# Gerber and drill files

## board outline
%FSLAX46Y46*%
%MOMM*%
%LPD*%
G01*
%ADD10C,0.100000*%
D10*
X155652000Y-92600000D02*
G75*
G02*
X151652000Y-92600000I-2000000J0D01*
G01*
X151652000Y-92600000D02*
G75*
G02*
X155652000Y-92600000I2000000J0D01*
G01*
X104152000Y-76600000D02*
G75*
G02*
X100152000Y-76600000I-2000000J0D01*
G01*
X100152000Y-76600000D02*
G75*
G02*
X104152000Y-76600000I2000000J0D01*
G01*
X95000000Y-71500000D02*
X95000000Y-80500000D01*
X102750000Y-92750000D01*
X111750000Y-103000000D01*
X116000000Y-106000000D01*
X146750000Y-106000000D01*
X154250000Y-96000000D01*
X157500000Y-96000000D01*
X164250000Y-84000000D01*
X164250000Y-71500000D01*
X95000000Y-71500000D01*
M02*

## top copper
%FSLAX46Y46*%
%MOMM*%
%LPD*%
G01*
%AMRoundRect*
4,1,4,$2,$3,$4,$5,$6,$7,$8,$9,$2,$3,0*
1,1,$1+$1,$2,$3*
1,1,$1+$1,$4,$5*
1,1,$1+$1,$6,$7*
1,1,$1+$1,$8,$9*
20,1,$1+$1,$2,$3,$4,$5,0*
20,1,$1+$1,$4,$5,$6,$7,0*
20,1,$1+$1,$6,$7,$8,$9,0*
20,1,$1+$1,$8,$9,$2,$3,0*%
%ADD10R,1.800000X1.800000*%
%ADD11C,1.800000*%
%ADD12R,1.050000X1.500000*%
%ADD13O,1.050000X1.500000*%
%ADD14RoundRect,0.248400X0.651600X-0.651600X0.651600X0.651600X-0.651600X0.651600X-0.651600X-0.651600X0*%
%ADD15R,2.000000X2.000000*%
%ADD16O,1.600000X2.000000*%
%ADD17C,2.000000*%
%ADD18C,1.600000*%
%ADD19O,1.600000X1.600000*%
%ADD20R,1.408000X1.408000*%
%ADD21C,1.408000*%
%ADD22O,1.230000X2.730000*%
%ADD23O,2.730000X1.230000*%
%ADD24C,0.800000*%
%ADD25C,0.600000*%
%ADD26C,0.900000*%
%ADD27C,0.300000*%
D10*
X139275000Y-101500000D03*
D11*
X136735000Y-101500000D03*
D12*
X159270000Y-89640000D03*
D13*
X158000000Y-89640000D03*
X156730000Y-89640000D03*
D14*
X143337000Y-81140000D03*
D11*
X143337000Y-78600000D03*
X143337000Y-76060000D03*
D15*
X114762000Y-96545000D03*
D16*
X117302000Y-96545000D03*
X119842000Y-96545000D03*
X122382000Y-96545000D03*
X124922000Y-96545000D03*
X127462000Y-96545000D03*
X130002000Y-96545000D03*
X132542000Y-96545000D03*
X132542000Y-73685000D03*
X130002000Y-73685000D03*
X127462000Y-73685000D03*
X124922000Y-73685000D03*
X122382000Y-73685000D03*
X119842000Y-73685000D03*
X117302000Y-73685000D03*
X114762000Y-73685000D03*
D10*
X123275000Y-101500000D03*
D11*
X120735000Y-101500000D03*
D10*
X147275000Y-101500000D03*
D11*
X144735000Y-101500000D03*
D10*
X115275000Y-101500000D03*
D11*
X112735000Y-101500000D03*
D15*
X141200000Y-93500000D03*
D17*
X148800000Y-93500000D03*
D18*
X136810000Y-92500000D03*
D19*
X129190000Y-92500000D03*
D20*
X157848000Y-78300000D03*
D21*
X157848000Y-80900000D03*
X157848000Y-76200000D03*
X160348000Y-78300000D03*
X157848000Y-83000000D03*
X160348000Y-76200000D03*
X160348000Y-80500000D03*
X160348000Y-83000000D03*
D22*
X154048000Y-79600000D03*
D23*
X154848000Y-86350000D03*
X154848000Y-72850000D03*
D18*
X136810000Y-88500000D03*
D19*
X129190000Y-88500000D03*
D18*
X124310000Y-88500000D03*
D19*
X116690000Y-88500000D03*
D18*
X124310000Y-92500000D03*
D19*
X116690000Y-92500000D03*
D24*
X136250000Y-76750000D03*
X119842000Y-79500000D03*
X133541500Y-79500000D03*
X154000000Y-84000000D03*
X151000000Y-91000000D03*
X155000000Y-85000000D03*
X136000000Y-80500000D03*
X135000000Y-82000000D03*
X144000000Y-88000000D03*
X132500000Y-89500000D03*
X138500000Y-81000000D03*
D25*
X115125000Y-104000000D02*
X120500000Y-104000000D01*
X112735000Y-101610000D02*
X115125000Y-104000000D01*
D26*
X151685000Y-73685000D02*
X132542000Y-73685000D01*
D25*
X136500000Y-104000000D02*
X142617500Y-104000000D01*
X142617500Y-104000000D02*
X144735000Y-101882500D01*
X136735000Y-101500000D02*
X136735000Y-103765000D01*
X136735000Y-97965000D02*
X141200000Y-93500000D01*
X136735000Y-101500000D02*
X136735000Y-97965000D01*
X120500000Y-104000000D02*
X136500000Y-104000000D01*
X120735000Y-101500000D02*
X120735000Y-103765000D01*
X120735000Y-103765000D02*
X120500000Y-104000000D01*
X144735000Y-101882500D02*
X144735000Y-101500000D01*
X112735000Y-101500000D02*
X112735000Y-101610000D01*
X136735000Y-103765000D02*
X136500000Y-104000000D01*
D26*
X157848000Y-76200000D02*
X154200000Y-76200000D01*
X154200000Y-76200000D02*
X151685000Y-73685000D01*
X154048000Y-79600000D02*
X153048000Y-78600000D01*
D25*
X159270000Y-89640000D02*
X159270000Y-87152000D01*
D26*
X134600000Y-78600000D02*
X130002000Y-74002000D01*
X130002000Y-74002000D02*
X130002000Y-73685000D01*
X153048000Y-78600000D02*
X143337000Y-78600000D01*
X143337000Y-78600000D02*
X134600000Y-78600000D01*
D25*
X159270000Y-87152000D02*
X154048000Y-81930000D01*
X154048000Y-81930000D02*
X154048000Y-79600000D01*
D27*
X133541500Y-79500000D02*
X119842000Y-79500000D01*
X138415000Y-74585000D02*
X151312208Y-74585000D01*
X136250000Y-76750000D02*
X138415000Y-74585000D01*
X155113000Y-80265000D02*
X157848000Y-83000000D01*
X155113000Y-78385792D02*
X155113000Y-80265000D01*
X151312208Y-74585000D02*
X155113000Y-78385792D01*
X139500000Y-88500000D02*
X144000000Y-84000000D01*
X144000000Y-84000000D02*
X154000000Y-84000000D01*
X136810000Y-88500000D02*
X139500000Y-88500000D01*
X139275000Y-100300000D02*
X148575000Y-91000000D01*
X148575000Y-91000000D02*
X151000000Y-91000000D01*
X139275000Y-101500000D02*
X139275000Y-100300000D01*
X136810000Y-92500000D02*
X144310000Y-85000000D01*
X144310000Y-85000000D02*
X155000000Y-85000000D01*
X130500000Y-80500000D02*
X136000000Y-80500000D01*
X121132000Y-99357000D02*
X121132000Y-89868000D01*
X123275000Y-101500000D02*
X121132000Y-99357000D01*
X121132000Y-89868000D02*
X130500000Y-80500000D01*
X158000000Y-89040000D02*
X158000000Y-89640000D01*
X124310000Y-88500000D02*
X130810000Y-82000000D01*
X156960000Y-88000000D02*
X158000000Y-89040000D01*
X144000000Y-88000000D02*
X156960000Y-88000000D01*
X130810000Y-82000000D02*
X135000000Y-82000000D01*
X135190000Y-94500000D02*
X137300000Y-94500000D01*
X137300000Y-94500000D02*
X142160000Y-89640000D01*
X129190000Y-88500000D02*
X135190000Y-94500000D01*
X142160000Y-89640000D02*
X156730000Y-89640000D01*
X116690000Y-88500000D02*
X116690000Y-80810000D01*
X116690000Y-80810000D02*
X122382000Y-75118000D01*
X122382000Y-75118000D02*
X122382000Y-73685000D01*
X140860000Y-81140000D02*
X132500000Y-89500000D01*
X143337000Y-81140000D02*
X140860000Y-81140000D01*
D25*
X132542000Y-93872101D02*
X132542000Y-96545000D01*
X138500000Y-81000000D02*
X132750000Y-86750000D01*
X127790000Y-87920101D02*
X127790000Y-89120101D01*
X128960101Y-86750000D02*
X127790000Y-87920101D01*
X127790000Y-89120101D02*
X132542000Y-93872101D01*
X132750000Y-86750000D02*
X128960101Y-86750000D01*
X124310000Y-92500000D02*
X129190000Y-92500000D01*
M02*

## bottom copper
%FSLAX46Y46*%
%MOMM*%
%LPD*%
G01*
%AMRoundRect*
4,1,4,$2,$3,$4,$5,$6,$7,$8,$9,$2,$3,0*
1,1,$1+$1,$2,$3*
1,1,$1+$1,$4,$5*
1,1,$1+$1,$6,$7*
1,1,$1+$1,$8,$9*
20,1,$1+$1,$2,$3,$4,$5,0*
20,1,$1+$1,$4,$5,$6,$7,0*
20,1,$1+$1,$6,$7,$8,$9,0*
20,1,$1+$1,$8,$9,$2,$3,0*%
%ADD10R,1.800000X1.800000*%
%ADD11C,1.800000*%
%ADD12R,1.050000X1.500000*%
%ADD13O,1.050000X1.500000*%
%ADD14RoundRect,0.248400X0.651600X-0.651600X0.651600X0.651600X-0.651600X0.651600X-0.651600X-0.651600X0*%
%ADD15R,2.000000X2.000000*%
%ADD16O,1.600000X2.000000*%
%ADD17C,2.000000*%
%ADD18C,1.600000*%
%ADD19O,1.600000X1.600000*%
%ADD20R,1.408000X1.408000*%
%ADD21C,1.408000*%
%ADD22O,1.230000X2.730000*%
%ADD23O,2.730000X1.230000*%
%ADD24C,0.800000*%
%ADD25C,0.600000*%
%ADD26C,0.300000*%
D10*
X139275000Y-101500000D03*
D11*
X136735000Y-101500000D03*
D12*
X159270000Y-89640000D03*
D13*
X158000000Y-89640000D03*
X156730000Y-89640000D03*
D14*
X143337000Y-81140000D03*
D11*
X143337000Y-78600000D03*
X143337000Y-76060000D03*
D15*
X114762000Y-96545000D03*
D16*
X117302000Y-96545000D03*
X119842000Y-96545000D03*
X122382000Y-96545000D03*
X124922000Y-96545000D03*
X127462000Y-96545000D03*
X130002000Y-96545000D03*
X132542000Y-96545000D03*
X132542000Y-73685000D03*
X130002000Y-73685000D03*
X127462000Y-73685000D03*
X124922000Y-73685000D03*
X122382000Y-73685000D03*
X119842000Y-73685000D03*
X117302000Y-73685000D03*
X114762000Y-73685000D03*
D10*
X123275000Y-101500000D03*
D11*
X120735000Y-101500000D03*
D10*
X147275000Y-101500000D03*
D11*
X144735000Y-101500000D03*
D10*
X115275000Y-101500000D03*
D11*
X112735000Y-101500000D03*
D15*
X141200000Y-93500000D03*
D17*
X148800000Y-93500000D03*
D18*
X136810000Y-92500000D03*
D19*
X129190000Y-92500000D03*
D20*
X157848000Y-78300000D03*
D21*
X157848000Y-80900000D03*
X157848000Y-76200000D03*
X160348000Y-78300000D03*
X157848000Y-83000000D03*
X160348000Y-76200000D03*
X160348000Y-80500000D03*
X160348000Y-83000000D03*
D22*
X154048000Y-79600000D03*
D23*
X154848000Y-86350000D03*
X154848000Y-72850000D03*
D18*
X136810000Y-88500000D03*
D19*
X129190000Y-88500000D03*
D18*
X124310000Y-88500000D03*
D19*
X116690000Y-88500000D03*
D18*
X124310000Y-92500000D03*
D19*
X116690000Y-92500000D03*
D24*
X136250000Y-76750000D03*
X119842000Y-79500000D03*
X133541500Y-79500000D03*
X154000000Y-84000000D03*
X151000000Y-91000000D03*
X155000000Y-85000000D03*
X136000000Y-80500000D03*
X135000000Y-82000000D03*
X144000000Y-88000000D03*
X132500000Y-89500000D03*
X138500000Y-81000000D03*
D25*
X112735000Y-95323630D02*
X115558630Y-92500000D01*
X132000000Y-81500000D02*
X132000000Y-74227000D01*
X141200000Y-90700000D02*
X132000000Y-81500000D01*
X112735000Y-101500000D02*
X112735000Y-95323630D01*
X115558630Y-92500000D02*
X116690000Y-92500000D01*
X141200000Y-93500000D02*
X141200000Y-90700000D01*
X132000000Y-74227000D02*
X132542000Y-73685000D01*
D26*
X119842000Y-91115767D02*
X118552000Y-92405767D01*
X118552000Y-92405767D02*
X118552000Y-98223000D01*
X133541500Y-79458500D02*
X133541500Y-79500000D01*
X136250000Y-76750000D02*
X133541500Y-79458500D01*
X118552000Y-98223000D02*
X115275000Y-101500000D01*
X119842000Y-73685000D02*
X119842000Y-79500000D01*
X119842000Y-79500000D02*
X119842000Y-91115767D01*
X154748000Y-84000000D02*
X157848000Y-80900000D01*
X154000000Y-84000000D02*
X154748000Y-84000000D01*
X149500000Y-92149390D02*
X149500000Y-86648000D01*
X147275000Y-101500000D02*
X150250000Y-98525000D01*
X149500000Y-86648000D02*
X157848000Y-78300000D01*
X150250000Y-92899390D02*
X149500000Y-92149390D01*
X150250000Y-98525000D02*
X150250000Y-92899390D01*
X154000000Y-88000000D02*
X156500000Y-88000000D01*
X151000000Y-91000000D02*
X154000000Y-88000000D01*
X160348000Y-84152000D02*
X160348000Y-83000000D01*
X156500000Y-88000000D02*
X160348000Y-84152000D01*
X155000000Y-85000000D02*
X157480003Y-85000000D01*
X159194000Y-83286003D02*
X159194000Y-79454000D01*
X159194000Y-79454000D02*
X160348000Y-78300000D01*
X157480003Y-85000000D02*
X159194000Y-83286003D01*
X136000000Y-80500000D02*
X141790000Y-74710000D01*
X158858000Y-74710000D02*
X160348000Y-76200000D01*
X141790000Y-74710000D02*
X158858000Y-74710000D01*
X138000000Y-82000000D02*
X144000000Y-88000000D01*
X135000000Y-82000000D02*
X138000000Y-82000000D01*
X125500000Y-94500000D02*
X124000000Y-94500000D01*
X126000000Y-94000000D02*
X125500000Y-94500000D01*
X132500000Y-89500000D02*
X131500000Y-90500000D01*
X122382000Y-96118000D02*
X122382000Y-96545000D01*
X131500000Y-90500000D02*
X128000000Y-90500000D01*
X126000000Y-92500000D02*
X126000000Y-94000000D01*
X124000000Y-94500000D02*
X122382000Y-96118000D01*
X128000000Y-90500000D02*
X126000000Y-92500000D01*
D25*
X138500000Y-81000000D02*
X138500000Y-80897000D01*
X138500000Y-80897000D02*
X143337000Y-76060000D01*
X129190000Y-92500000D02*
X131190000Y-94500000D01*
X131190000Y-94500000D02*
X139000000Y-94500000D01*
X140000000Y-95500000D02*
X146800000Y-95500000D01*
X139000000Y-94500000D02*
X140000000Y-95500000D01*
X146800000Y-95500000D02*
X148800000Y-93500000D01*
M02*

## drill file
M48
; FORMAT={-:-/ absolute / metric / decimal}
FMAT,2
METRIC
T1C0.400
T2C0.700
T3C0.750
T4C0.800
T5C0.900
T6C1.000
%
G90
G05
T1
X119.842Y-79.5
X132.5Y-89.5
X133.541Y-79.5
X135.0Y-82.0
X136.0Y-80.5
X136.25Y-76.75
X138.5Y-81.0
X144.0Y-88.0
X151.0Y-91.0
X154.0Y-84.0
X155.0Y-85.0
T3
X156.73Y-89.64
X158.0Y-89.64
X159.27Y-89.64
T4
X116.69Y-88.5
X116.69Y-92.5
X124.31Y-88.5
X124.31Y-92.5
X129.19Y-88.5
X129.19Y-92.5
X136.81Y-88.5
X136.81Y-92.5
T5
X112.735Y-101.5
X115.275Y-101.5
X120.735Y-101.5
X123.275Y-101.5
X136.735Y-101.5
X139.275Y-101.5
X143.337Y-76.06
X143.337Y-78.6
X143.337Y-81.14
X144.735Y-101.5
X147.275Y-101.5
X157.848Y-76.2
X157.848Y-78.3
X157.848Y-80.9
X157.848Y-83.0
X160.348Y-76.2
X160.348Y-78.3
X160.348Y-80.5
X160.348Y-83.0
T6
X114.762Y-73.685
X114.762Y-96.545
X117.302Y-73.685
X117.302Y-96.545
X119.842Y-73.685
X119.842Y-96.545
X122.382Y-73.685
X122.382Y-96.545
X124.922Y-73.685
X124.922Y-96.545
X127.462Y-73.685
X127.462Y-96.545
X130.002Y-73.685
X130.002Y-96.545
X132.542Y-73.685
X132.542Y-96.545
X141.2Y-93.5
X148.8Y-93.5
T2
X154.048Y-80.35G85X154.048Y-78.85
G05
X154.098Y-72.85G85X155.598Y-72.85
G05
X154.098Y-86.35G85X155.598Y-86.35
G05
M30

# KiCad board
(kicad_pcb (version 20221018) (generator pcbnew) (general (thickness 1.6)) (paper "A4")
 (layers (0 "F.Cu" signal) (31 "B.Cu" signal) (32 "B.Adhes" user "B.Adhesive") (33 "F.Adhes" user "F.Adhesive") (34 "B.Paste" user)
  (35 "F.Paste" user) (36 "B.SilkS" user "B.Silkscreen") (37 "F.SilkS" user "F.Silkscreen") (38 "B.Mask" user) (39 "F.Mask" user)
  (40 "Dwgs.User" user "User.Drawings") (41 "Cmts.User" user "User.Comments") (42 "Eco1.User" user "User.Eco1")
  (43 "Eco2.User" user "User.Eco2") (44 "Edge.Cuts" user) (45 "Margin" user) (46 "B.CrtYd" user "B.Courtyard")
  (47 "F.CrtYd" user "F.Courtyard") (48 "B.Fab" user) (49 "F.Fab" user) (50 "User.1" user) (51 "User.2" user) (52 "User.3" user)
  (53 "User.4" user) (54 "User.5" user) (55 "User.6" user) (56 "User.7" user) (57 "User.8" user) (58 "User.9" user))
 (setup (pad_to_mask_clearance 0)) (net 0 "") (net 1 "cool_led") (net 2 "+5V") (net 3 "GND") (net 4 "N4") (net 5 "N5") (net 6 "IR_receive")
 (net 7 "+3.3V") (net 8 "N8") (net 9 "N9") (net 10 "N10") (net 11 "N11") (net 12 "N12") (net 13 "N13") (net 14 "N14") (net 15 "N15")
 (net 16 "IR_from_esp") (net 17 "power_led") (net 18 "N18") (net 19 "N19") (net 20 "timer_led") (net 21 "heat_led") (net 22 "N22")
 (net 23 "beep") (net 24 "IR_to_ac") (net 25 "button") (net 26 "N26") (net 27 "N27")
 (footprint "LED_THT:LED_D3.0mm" (layer "F.Cu") (at 139.275 101.5 180)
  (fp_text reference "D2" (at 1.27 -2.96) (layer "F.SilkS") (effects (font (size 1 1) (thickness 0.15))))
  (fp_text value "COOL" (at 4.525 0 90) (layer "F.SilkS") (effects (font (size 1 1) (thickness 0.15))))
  (pad "1" thru_hole rect (at 0 0 180) (size 1.8 1.8) (drill 0.9) (layers "*.Cu" "*.Mask") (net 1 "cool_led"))
  (pad "2" thru_hole circle (at 2.54 0 180) (size 1.8 1.8) (drill 0.9) (layers "*.Cu" "*.Mask") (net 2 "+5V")))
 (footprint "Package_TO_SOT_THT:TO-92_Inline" (layer "F.Cu") (at 159.27 89.64 180)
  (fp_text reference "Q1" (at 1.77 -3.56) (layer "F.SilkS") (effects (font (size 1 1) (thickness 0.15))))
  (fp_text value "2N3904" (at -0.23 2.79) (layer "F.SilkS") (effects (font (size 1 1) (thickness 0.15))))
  (pad "1" thru_hole rect (at 0 0 180) (size 1.05 1.5) (drill 0.75) (layers "*.Cu" "*.Mask") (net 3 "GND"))
  (pad "2" thru_hole oval (at 1.27 0 180) (size 1.05 1.5) (drill 0.75) (layers "*.Cu" "*.Mask") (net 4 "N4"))
  (pad "3" thru_hole oval (at 2.54 0 180) (size 1.05 1.5) (drill 0.75) (layers "*.Cu" "*.Mask") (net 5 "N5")))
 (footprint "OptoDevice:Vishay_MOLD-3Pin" (layer "F.Cu") (at 143.337 81.14 90)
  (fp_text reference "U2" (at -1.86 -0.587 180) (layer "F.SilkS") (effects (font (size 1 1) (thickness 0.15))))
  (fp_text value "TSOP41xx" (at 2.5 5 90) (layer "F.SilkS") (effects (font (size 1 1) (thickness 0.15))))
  (pad "1" thru_hole roundrect (at 0 0 90) (size 1.8 1.8) (drill 0.9) (layers "*.Cu" "*.Mask") (roundrect_rratio 0.138) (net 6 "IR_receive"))
  (pad "2" thru_hole circle (at 2.54 0 90) (size 1.8 1.8) (drill 0.9) (layers "*.Cu" "*.Mask") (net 3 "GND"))
  (pad "3" thru_hole circle (at 5.08 0 90) (size 1.8 1.8) (drill 0.9) (layers "*.Cu" "*.Mask") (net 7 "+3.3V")))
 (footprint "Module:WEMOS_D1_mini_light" (layer "F.Cu") (at 114.762 96.545 90)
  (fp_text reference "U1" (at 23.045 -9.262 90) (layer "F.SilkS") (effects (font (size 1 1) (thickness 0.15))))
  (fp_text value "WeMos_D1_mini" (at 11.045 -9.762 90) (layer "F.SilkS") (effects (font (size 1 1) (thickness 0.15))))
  (pad "1" thru_hole rect (at 0 0 90) (size 2 2) (drill 1) (layers "*.Cu" "*.Mask") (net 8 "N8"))
  (pad "2" thru_hole oval (at 0 2.54 90) (size 2 1.6) (drill 1) (layers "*.Cu" "*.Mask") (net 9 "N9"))
  (pad "3" thru_hole oval (at 0 5.08 90) (size 2 1.6) (drill 1) (layers "*.Cu" "*.Mask") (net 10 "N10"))
  (pad "4" thru_hole oval (at 0 7.62 90) (size 2 1.6) (drill 1) (layers "*.Cu" "*.Mask") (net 6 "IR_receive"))
  (pad "5" thru_hole oval (at 0 10.16 90) (size 2 1.6) (drill 1) (layers "*.Cu" "*.Mask") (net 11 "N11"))
  (pad "6" thru_hole oval (at 0 12.7 90) (size 2 1.6) (drill 1) (layers "*.Cu" "*.Mask") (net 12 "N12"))
  (pad "7" thru_hole oval (at 0 15.24 90) (size 2 1.6) (drill 1) (layers "*.Cu" "*.Mask") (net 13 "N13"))
  (pad "8" thru_hole oval (at 0 17.78 90) (size 2 1.6) (drill 1) (layers "*.Cu" "*.Mask") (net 7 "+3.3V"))
  (pad "9" thru_hole oval (at 22.86 17.78 90) (size 2 1.6) (drill 1) (layers "*.Cu" "*.Mask") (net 2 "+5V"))
  (pad "10" thru_hole oval (at 22.86 15.24 90) (size 2 1.6) (drill 1) (layers "*.Cu" "*.Mask") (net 3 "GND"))
  (pad "11" thru_hole oval (at 22.86 12.7 90) (size 2 1.6) (drill 1) (layers "*.Cu" "*.Mask") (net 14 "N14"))
  (pad "12" thru_hole oval (at 22.86 10.16 90) (size 2 1.6) (drill 1) (layers "*.Cu" "*.Mask") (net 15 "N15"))
  (pad "13" thru_hole oval (at 22.86 7.62 90) (size 2 1.6) (drill 1) (layers "*.Cu" "*.Mask") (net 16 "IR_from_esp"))
  (pad "14" thru_hole oval (at 22.86 5.08 90) (size 2 1.6) (drill 1) (layers "*.Cu" "*.Mask") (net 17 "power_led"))
  (pad "15" thru_hole oval (at 22.86 2.54 90) (size 2 1.6) (drill 1) (layers "*.Cu" "*.Mask") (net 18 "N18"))
  (pad "16" thru_hole oval (at 22.86 0 90) (size 2 1.6) (drill 1) (layers "*.Cu" "*.Mask") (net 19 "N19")))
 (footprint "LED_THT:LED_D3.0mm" (layer "F.Cu") (at 123.275 101.5 180)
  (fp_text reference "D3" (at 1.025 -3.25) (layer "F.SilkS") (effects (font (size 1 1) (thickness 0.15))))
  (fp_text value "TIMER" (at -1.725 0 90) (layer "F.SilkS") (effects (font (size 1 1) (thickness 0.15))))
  (pad "1" thru_hole rect (at 0 0 180) (size 1.8 1.8) (drill 0.9) (layers "*.Cu" "*.Mask") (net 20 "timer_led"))
  (pad "2" thru_hole circle (at 2.54 0 180) (size 1.8 1.8) (drill 0.9) (layers "*.Cu" "*.Mask") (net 2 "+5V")))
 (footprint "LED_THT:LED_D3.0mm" (layer "F.Cu") (at 147.275 101.5 180)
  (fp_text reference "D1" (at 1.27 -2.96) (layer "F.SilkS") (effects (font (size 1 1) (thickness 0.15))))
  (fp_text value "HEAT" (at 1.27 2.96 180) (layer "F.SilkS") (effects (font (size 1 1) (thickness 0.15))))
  (pad "1" thru_hole rect (at 0 0 180) (size 1.8 1.8) (drill 0.9) (layers "*.Cu" "*.Mask") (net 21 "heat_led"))
  (pad "2" thru_hole circle (at 2.54 0 180) (size 1.8 1.8) (drill 0.9) (layers "*.Cu" "*.Mask") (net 2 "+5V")))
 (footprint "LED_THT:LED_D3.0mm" (layer "F.Cu") (at 115.275 101.5 180)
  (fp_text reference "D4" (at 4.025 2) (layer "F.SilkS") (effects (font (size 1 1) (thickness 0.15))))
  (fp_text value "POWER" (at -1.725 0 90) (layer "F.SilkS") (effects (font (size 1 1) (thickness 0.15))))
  (pad "1" thru_hole rect (at 0 0 180) (size 1.8 1.8) (drill 0.9) (layers "*.Cu" "*.Mask") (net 17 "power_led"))
  (pad "2" thru_hole circle (at 2.54 0 180) (size 1.8 1.8) (drill 0.9) (layers "*.Cu" "*.Mask") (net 2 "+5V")))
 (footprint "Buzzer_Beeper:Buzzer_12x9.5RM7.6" (layer "B.Cu") (at 141.2 93.5)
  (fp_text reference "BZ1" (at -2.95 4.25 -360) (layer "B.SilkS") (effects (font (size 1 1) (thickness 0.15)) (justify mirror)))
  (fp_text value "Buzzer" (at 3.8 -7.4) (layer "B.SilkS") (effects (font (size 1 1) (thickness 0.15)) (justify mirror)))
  (pad "1" thru_hole rect (at 0 0) (size 2 2) (drill 1) (layers "*.Cu" "*.Mask") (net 2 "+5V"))
  (pad "2" thru_hole circle (at 7.6 0) (size 2 2) (drill 1) (layers "*.Cu" "*.Mask") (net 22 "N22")))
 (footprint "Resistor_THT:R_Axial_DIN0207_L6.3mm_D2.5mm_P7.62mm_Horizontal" (layer "B.Cu") (at 136.81 92.5 180)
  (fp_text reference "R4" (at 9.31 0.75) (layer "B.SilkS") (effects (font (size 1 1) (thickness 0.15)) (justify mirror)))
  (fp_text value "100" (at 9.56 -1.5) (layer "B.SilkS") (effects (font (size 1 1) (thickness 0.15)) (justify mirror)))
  (pad "1" thru_hole circle (at 0 0 180) (size 1.6 1.6) (drill 0.8) (layers "*.Cu" "*.Mask") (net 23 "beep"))
  (pad "2" thru_hole oval (at 7.62 0 180) (size 1.6 1.6) (drill 0.8) (layers "*.Cu" "*.Mask") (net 22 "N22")))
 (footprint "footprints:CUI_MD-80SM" (layer "B.Cu") (at 154.048 79.6 90)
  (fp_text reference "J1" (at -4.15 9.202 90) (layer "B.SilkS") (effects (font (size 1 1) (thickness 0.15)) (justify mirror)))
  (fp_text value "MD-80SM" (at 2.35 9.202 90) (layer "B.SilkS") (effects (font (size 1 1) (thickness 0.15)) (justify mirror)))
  (pad "1" thru_hole rect (at 1.3 3.8 90) (size 1.408 1.408) (drill 0.9) (layers "*.Cu" "*.Mask") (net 21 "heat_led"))
  (pad "2" thru_hole circle (at -1.3 3.8 90) (size 1.408 1.408) (drill 0.9) (layers "*.Cu" "*.Mask") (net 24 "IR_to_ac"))
  (pad "3" thru_hole circle (at 3.4 3.8 90) (size 1.408 1.408) (drill 0.9) (layers "*.Cu" "*.Mask") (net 2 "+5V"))
  (pad "4" thru_hole circle (at 1.3 6.3 90) (size 1.408 1.408) (drill 0.9) (layers "*.Cu" "*.Mask") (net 23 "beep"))
  (pad "5" thru_hole circle (at -3.4 3.8 90) (size 1.408 1.408) (drill 0.9) (layers "*.Cu" "*.Mask") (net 17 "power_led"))
  (pad "6" thru_hole circle (at 3.4 6.3 90) (size 1.408 1.408) (drill 0.9) (layers "*.Cu" "*.Mask") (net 20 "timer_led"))
  (pad "7" thru_hole circle (at -0.9 6.3 90) (size 1.408 1.408) (drill 0.9) (layers "*.Cu" "*.Mask") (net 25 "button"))
  (pad "8" thru_hole circle (at -3.4 6.3 90) (size 1.408 1.408) (drill 0.9) (layers "*.Cu" "*.Mask") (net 1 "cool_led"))
  (pad "S1" thru_hole oval (at 0 0 90) (size 2.73 1.23) (drill oval 2.2 0.7) (layers "*.Cu" "*.Mask") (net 3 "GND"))
  (pad "S2" thru_hole oval (at -6.75 0.8 90) (size 1.23 2.73) (drill oval 0.7 2.2) (layers "*.Cu" "*.Mask") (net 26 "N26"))
  (pad "S3" thru_hole oval (at 6.75 0.8 90) (size 1.23 2.73) (drill oval 0.7 2.2) (layers "*.Cu" "*.Mask") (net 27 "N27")))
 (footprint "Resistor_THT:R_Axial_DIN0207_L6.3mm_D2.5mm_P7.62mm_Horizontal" (layer "B.Cu") (at 136.81 88.5 180)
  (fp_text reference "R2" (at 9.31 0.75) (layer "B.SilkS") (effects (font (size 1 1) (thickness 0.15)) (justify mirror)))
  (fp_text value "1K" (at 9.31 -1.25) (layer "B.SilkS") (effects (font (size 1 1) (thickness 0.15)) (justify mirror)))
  (pad "1" thru_hole circle (at 0 0 180) (size 1.6 1.6) (drill 0.8) (layers "*.Cu" "*.Mask") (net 24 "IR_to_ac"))
  (pad "2" thru_hole oval (at 7.62 0 180) (size 1.6 1.6) (drill 0.8) (layers "*.Cu" "*.Mask") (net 5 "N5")))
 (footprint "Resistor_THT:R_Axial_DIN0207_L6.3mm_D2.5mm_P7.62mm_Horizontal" (layer "B.Cu") (at 124.31 88.5 180)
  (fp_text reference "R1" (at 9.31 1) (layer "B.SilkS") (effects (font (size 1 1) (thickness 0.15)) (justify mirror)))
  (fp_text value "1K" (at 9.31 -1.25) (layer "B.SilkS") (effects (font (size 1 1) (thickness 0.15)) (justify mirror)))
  (pad "1" thru_hole circle (at 0 0 180) (size 1.6 1.6) (drill 0.8) (layers "*.Cu" "*.Mask") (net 4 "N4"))
  (pad "2" thru_hole oval (at 7.62 0 180) (size 1.6 1.6) (drill 0.8) (layers "*.Cu" "*.Mask") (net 16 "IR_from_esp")))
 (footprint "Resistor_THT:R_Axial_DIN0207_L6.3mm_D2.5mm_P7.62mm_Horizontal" (layer "B.Cu") (at 124.31 92.5 180)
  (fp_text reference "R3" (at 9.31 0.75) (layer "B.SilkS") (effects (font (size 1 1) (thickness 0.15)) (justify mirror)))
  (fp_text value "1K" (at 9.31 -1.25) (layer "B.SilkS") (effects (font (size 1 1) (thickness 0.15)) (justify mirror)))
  (pad "1" thru_hole circle (at 0 0 180) (size 1.6 1.6) (drill 0.8) (layers "*.Cu" "*.Mask") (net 22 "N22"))
  (pad "2" thru_hole oval (at 7.62 0 180) (size 1.6 1.6) (drill 0.8) (layers "*.Cu" "*.Mask") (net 2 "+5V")))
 (gr_circle (center 153.652 92.6) (end 155.652 92.6) (stroke (width 0.1) (type default)) (fill none) (layer "Edge.Cuts"))
 (gr_circle (center 102.152 76.6) (end 104.152 76.6) (stroke (width 0.1) (type default)) (fill none) (layer "Edge.Cuts"))
 (gr_poly
  (pts (xy 95 71.5) (xy 95 80.5) (xy 102.75 92.75) (xy 111.75 103) (xy 116 106) (xy 146.75 106) (xy 154.25 96) (xy 157.5 96) (xy 164.25 84)
   (xy 164.25 71.5))
  (stroke (width 0.1) (type solid)) (fill none) (layer "Edge.Cuts"))
 (segment (start 115.125 104) (end 120.5 104) (width 0.6) (layer "F.Cu") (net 2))
 (segment (start 112.735 101.61) (end 115.125 104) (width 0.6) (layer "F.Cu") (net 2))
 (segment (start 151.685 73.685) (end 132.542 73.685) (width 0.9) (layer "F.Cu") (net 2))
 (segment (start 136.5 104) (end 142.6175 104) (width 0.6) (layer "F.Cu") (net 2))
 (segment (start 142.6175 104) (end 144.735 101.8825) (width 0.6) (layer "F.Cu") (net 2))
 (segment (start 136.735 101.5) (end 136.735 103.765) (width 0.6) (layer "F.Cu") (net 2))
 (segment (start 136.735 97.965) (end 141.2 93.5) (width 0.6) (layer "F.Cu") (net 2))
 (segment (start 136.735 101.5) (end 136.735 97.965) (width 0.6) (layer "F.Cu") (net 2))
 (segment (start 120.5 104) (end 136.5 104) (width 0.6) (layer "F.Cu") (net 2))
 (segment (start 120.735 101.5) (end 120.735 103.765) (width 0.6) (layer "F.Cu") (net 2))
 (segment (start 120.735 103.765) (end 120.5 104) (width 0.6) (layer "F.Cu") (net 2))
 (segment (start 144.735 101.8825) (end 144.735 101.5) (width 0.6) (layer "F.Cu") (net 2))
 (segment (start 112.735 101.5) (end 112.735 101.61) (width 0.6) (layer "F.Cu") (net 2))
 (segment (start 136.735 103.765) (end 136.5 104) (width 0.6) (layer "F.Cu") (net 2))
 (segment (start 157.848 76.2) (end 154.2 76.2) (width 0.9) (layer "F.Cu") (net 2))
 (segment (start 154.2 76.2) (end 151.685 73.685) (width 0.9) (layer "F.Cu") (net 2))
 (segment (start 112.735 95.32363) (end 115.55863 92.5) (width 0.6) (layer "B.Cu") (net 2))
 (segment (start 132 81.5) (end 132 74.227) (width 0.6) (layer "B.Cu") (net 2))
 (segment (start 141.2 90.7) (end 132 81.5) (width 0.6) (layer "B.Cu") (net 2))
 (segment (start 112.735 101.5) (end 112.735 95.32363) (width 0.6) (layer "B.Cu") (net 2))
 (segment (start 115.55863 92.5) (end 116.69 92.5) (width 0.6) (layer "B.Cu") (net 2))
 (segment (start 141.2 93.5) (end 141.2 90.7) (width 0.6) (layer "B.Cu") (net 2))
 (segment (start 132 74.227) (end 132.542 73.685) (width 0.6) (layer "B.Cu") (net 2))
 (segment (start 154.048 79.6) (end 153.048 78.6) (width 0.9) (layer "F.Cu") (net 3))
 (segment (start 159.27 89.64) (end 159.27 87.152) (width 0.6) (layer "F.Cu") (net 3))
 (segment (start 134.6 78.6) (end 130.002 74.002) (width 0.9) (layer "F.Cu") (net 3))
 (segment (start 130.002 74.002) (end 130.002 73.685) (width 0.9) (layer "F.Cu") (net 3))
 (segment (start 153.048 78.6) (end 143.337 78.6) (width 0.9) (layer "F.Cu") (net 3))
 (segment (start 143.337 78.6) (end 134.6 78.6) (width 0.9) (layer "F.Cu") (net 3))
 (segment (start 159.27 87.152) (end 154.048 81.93) (width 0.6) (layer "F.Cu") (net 3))
 (segment (start 154.048 81.93) (end 154.048 79.6) (width 0.6) (layer "F.Cu") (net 3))
 (segment (start 133.5415 79.5) (end 119.842 79.5) (width 0.3) (layer "F.Cu") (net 17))
 (segment (start 138.415 74.585) (end 151.312208 74.585) (width 0.3) (layer "F.Cu") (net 17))
 (segment (start 136.25 76.75) (end 138.415 74.585) (width 0.3) (layer "F.Cu") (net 17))
 (segment (start 155.113 80.265) (end 157.848 83) (width 0.3) (layer "F.Cu") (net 17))
 (segment (start 155.113 78.385792) (end 155.113 80.265) (width 0.3) (layer "F.Cu") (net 17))
 (segment (start 151.312208 74.585) (end 155.113 78.385792) (width 0.3) (layer "F.Cu") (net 17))
 (via (at 136.25 76.75) (size 0.8) (drill 0.4) (layers "F.Cu" "B.Cu") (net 17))
 (via (at 119.842 79.5) (size 0.8) (drill 0.4) (layers "F.Cu" "B.Cu") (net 17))
 (via (at 133.5415 79.5) (size 0.8) (drill 0.4) (layers "F.Cu" "B.Cu") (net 17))
 (segment (start 119.842 91.115767) (end 118.552 92.405767) (width 0.3) (layer "B.Cu") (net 17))
 (segment (start 118.552 92.405767) (end 118.552 98.223) (width 0.3) (layer "B.Cu") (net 17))
 (segment (start 133.5415 79.4585) (end 133.5415 79.5) (width 0.3) (layer "B.Cu") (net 17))
 (segment (start 136.25 76.75) (end 133.5415 79.4585) (width 0.3) (layer "B.Cu") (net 17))
 (segment (start 118.552 98.223) (end 115.275 101.5) (width 0.3) (layer "B.Cu") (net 17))
 (segment (start 119.842 73.685) (end 119.842 79.5) (width 0.3) (layer "B.Cu") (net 17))
 (segment (start 119.842 79.5) (end 119.842 91.115767) (width 0.3) (layer "B.Cu") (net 17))
 (segment (start 139.5 88.5) (end 144 84) (width 0.3) (layer "F.Cu") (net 24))
 (segment (start 144 84) (end 154 84) (width 0.3) (layer "F.Cu") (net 24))
 (segment (start 136.81 88.5) (end 139.5 88.5) (width 0.3) (layer "F.Cu") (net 24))
 (via (at 154 84) (size 0.8) (drill 0.4) (layers "F.Cu" "B.Cu") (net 24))
 (segment (start 154.748 84) (end 157.848 80.9) (width 0.3) (layer "B.Cu") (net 24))
 (segment (start 154 84) (end 154.748 84) (width 0.3) (layer "B.Cu") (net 24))
 (segment (start 149.5 92.14939) (end 149.5 86.648) (width 0.3) (layer "B.Cu") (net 21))
 (segment (start 147.275 101.5) (end 150.25 98.525) (width 0.3) (layer "B.Cu") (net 21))
 (segment (start 149.5 86.648) (end 157.848 78.3) (width 0.3) (layer "B.Cu") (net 21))
 (segment (start 150.25 92.89939) (end 149.5 92.14939) (width 0.3) (layer "B.Cu") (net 21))
 (segment (start 150.25 98.525) (end 150.25 92.89939) (width 0.3) (layer "B.Cu") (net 21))
 (segment (start 139.275 100.3) (end 148.575 91) (width 0.3) (layer "F.Cu") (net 1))
 (segment (start 148.575 91) (end 151 91) (width 0.3) (layer "F.Cu") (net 1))
 (segment (start 139.275 101.5) (end 139.275 100.3) (width 0.3) (layer "F.Cu") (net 1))
 (via (at 151 91) (size 0.8) (drill 0.4) (layers "F.Cu" "B.Cu") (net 1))
 (segment (start 154 88) (end 156.5 88) (width 0.3) (layer "B.Cu") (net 1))
 (segment (start 151 91) (end 154 88) (width 0.3) (layer "B.Cu") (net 1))
 (segment (start 160.348 84.152) (end 160.348 83) (width 0.3) (layer "B.Cu") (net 1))
 (segment (start 156.5 88) (end 160.348 84.152) (width 0.3) (layer "B.Cu") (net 1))
 (segment (start 136.81 92.5) (end 144.31 85) (width 0.3) (layer "F.Cu") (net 23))
 (segment (start 144.31 85) (end 155 85) (width 0.3) (layer "F.Cu") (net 23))
 (via (at 155 85) (size 0.8) (drill 0.4) (layers "F.Cu" "B.Cu") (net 23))
 (segment (start 155 85) (end 157.480003 85) (width 0.3) (layer "B.Cu") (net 23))
 (segment (start 159.194 83.286003) (end 159.194 79.454) (width 0.3) (layer "B.Cu") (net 23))
 (segment (start 159.194 79.454) (end 160.348 78.3) (width 0.3) (layer "B.Cu") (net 23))
 (segment (start 157.480003 85) (end 159.194 83.286003) (width 0.3) (layer "B.Cu") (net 23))
 (segment (start 130.5 80.5) (end 136 80.5) (width 0.3) (layer "F.Cu") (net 20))
 (segment (start 121.132 99.357) (end 121.132 89.868) (width 0.3) (layer "F.Cu") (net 20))
 (segment (start 123.275 101.5) (end 121.132 99.357) (width 0.3) (layer "F.Cu") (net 20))
 (segment (start 121.132 89.868) (end 130.5 80.5) (width 0.3) (layer "F.Cu") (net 20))
 (via (at 136 80.5) (size 0.8) (drill 0.4) (layers "F.Cu" "B.Cu") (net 20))
 (segment (start 136 80.5) (end 141.79 74.71) (width 0.3) (layer "B.Cu") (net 20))
 (segment (start 158.858 74.71) (end 160.348 76.2) (width 0.3) (layer "B.Cu") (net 20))
 (segment (start 141.79 74.71) (end 158.858 74.71) (width 0.3) (layer "B.Cu") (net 20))
 (segment (start 158 89.04) (end 158 89.64) (width 0.3) (layer "F.Cu") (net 4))
 (segment (start 124.31 88.5) (end 130.81 82) (width 0.3) (layer "F.Cu") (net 4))
 (segment (start 156.96 88) (end 158 89.04) (width 0.3) (layer "F.Cu") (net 4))
 (segment (start 144 88) (end 156.96 88) (width 0.3) (layer "F.Cu") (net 4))
 (segment (start 130.81 82) (end 135 82) (width 0.3) (layer "F.Cu") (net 4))
 (via (at 135 82) (size 0.8) (drill 0.4) (layers "F.Cu" "B.Cu") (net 4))
 (via (at 144 88) (size 0.8) (drill 0.4) (layers "F.Cu" "B.Cu") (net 4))
 (segment (start 138 82) (end 144 88) (width 0.3) (layer "B.Cu") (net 4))
 (segment (start 135 82) (end 138 82) (width 0.3) (layer "B.Cu") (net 4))
 (segment (start 135.19 94.5) (end 137.3 94.5) (width 0.3) (layer "F.Cu") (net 5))
 (segment (start 137.3 94.5) (end 142.16 89.64) (width 0.3) (layer "F.Cu") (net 5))
 (segment (start 129.19 88.5) (end 135.19 94.5) (width 0.3) (layer "F.Cu") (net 5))
 (segment (start 142.16 89.64) (end 156.73 89.64) (width 0.3) (layer "F.Cu") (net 5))
 (segment (start 116.69 88.5) (end 116.69 80.81) (width 0.3) (layer "F.Cu") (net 16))
 (segment (start 116.69 80.81) (end 122.382 75.118) (width 0.3) (layer "F.Cu") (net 16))
 (segment (start 122.382 75.118) (end 122.382 73.685) (width 0.3) (layer "F.Cu") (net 16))
 (segment (start 140.86 81.14) (end 132.5 89.5) (width 0.3) (layer "F.Cu") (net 6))
 (segment (start 143.337 81.14) (end 140.86 81.14) (width 0.3) (layer "F.Cu") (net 6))
 (via (at 132.5 89.5) (size 0.8) (drill 0.4) (layers "F.Cu" "B.Cu") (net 6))
 (segment (start 125.5 94.5) (end 124 94.5) (width 0.3) (layer "B.Cu") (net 6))
 (segment (start 126 94) (end 125.5 94.5) (width 0.3) (layer "B.Cu") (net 6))
 (segment (start 132.5 89.5) (end 131.5 90.5) (width 0.3) (layer "B.Cu") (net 6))
 (segment (start 122.382 96.118) (end 122.382 96.545) (width 0.3) (layer "B.Cu") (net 6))
 (segment (start 131.5 90.5) (end 128 90.5) (width 0.3) (layer "B.Cu") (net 6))
 (segment (start 126 92.5) (end 126 94) (width 0.3) (layer "B.Cu") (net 6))
 (segment (start 124 94.5) (end 122.382 96.118) (width 0.3) (layer "B.Cu") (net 6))
 (segment (start 128 90.5) (end 126 92.5) (width 0.3) (layer "B.Cu") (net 6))
 (segment (start 132.542 93.872101) (end 132.542 96.545) (width 0.6) (layer "F.Cu") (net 7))
 (segment (start 138.5 81) (end 132.75 86.75) (width 0.6) (layer "F.Cu") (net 7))
 (segment (start 127.79 87.920101) (end 127.79 89.120101) (width 0.6) (layer "F.Cu") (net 7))
 (segment (start 128.960101 86.75) (end 127.79 87.920101) (width 0.6) (layer "F.Cu") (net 7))
 (segment (start 127.79 89.120101) (end 132.542 93.872101) (width 0.6) (layer "F.Cu") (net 7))
 (segment (start 132.75 86.75) (end 128.960101 86.75) (width 0.6) (layer "F.Cu") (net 7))
 (via (at 138.5 81) (size 0.8) (drill 0.4) (layers "F.Cu" "B.Cu") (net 7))
 (segment (start 138.5 81) (end 138.5 80.897) (width 0.6) (layer "B.Cu") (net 7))
 (segment (start 138.5 80.897) (end 143.337 76.06) (width 0.6) (layer "B.Cu") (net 7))
 (segment (start 124.31 92.5) (end 129.19 92.5) (width 0.6) (layer "F.Cu") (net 22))
 (segment (start 129.19 92.5) (end 131.19 94.5) (width 0.6) (layer "B.Cu") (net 22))
 (segment (start 131.19 94.5) (end 139 94.5) (width 0.6) (layer "B.Cu") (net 22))
 (segment (start 140 95.5) (end 146.8 95.5) (width 0.6) (layer "B.Cu") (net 22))
 (segment (start 139 94.5) (end 140 95.5) (width 0.6) (layer "B.Cu") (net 22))
 (segment (start 146.8 95.5) (end 148.8 93.5) (width 0.6) (layer "B.Cu") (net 22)))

